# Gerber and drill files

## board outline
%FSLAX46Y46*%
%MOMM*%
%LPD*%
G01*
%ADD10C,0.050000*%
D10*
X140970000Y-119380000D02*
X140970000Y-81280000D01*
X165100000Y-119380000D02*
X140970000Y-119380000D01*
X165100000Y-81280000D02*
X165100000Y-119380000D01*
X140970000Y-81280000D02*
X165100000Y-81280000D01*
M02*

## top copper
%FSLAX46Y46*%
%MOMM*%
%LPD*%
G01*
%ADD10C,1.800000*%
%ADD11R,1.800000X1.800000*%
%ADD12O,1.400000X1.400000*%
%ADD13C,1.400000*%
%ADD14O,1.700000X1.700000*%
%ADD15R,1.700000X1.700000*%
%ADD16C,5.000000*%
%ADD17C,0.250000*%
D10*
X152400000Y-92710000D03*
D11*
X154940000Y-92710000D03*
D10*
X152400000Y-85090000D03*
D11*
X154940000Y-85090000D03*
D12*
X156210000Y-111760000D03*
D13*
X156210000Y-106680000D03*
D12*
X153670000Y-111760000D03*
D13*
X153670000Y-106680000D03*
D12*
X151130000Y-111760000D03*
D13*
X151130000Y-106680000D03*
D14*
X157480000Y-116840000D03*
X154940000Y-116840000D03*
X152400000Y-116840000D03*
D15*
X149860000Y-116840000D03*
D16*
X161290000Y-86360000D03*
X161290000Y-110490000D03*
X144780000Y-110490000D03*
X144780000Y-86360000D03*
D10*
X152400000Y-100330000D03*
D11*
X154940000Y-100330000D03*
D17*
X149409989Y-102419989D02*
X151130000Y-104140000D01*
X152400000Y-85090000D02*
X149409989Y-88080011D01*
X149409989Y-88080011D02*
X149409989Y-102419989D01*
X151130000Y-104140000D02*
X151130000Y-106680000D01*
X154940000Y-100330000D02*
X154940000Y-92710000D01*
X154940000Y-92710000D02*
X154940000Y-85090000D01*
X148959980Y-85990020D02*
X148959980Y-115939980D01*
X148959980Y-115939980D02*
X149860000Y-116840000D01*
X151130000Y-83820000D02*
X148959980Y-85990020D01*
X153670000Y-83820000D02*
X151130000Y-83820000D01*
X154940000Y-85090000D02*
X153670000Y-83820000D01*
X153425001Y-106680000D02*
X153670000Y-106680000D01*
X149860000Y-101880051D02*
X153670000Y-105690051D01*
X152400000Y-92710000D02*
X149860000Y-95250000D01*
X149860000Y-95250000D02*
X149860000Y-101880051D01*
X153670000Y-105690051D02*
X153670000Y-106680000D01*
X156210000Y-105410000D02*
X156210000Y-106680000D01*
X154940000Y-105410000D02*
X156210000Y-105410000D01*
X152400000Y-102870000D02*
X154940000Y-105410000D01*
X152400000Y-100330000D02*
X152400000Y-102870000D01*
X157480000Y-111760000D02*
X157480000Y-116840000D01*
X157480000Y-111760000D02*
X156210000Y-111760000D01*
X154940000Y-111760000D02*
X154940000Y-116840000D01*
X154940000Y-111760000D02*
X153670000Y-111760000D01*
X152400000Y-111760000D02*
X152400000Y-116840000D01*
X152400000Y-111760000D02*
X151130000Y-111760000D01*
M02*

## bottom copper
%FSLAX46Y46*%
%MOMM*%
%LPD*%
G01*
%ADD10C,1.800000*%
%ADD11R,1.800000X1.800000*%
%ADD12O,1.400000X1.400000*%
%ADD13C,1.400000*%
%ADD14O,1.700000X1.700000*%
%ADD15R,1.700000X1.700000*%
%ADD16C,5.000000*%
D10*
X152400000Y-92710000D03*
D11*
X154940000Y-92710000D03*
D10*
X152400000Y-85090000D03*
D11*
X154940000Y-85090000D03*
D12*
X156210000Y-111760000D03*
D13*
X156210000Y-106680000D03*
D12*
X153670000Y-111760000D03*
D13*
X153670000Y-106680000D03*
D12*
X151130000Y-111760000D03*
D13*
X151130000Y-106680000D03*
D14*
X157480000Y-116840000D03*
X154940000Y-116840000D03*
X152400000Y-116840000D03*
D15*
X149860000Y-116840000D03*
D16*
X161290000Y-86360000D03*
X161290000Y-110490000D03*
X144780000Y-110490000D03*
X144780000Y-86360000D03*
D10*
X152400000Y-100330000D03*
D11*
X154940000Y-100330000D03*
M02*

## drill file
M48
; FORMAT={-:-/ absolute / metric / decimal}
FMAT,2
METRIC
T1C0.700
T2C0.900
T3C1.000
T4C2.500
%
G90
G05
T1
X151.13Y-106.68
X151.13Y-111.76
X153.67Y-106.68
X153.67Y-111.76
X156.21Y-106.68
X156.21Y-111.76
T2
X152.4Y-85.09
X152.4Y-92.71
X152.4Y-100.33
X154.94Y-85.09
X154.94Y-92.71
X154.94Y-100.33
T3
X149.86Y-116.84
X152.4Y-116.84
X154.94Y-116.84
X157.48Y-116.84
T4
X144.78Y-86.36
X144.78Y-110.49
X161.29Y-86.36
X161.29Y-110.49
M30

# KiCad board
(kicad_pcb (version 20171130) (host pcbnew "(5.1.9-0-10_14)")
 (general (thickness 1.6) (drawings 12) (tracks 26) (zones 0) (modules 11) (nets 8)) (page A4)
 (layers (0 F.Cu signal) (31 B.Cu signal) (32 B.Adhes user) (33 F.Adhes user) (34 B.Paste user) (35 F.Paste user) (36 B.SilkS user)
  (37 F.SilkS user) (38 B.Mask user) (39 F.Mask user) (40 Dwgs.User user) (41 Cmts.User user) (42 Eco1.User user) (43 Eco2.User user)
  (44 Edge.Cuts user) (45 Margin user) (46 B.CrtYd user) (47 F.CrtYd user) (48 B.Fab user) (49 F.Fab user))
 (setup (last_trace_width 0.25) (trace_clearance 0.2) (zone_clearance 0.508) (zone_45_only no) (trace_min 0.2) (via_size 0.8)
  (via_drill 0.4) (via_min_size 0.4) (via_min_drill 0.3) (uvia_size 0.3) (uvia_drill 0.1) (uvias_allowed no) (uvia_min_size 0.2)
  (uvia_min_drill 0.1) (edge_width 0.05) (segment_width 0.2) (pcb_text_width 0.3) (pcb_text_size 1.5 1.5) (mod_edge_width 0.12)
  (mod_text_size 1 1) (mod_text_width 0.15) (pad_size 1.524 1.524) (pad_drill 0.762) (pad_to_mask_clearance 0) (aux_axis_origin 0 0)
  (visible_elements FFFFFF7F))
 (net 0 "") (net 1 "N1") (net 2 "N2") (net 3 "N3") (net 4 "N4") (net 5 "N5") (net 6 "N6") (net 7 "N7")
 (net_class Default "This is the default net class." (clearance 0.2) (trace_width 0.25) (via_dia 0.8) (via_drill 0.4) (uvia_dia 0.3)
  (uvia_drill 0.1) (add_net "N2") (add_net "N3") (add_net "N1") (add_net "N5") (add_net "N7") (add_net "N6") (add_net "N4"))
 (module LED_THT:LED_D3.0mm (layer F.Cu) (at 154.94 92.71 180)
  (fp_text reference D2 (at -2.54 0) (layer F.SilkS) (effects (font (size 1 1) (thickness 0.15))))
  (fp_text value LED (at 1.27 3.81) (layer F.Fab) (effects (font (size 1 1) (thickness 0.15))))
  (pad 2 thru_hole circle (at 2.54 0 180) (size 1.8 1.8) (drill 0.9) (layers *.Cu *.Mask) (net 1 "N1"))
  (pad 1 thru_hole rect (at 0 0 180) (size 1.8 1.8) (drill 0.9) (layers *.Cu *.Mask) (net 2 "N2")))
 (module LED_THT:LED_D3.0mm (layer F.Cu) (at 154.94 85.09 180)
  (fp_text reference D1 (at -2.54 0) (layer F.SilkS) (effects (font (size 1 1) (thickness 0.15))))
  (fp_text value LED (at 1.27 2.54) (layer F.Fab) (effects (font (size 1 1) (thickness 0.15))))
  (pad 2 thru_hole circle (at 2.54 0 180) (size 1.8 1.8) (drill 0.9) (layers *.Cu *.Mask) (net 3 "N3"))
  (pad 1 thru_hole rect (at 0 0 180) (size 1.8 1.8) (drill 0.9) (layers *.Cu *.Mask) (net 2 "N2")))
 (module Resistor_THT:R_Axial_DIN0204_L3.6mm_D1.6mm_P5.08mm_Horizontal (layer F.Cu) (at 156.21 106.68 270)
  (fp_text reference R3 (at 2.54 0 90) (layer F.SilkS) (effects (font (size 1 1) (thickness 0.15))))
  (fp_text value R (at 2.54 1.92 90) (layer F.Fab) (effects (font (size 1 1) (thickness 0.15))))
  (pad 2 thru_hole oval (at 5.08 0 270) (size 1.4 1.4) (drill 0.7) (layers *.Cu *.Mask) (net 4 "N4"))
  (pad 1 thru_hole circle (at 0 0 270) (size 1.4 1.4) (drill 0.7) (layers *.Cu *.Mask) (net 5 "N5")))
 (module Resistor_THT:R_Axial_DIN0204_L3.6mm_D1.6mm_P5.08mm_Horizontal (layer F.Cu) (at 153.67 106.68 270)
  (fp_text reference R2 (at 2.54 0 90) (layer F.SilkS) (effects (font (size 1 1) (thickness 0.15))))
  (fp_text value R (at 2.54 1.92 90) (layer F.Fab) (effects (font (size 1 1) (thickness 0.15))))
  (pad 2 thru_hole oval (at 5.08 0 270) (size 1.4 1.4) (drill 0.7) (layers *.Cu *.Mask) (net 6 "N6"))
  (pad 1 thru_hole circle (at 0 0 270) (size 1.4 1.4) (drill 0.7) (layers *.Cu *.Mask) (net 1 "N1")))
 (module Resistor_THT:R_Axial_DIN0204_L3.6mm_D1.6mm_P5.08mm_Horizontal (layer F.Cu) (at 151.13 106.68 270)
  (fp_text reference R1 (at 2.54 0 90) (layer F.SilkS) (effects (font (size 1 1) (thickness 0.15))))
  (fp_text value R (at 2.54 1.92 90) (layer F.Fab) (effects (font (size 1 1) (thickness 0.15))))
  (pad 2 thru_hole oval (at 5.08 0 270) (size 1.4 1.4) (drill 0.7) (layers *.Cu *.Mask) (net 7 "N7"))
  (pad 1 thru_hole circle (at 0 0 270) (size 1.4 1.4) (drill 0.7) (layers *.Cu *.Mask) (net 3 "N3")))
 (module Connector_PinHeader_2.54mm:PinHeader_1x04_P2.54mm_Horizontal (layer B.Cu) (at 149.86 116.84 270)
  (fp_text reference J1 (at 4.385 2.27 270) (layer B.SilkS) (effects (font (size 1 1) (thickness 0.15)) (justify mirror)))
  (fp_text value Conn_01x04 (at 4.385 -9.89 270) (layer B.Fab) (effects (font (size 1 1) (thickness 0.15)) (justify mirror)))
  (pad 4 thru_hole oval (at 0 -7.62 270) (size 1.7 1.7) (drill 1) (layers *.Cu *.Mask) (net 4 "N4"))
  (pad 3 thru_hole oval (at 0 -5.08 270) (size 1.7 1.7) (drill 1) (layers *.Cu *.Mask) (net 6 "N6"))
  (pad 2 thru_hole oval (at 0 -2.54 270) (size 1.7 1.7) (drill 1) (layers *.Cu *.Mask) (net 7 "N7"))
  (pad 1 thru_hole rect (at 0 0 270) (size 1.7 1.7) (drill 1) (layers *.Cu *.Mask) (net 2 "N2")))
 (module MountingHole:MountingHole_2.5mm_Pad (layer F.Cu) (at 161.29 86.36)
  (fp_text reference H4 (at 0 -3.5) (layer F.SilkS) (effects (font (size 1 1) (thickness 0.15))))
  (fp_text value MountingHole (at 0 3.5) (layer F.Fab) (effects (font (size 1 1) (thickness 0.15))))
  (pad 1 thru_hole circle (at 0 0) (size 5 5) (drill 2.5) (layers *.Cu *.Mask)))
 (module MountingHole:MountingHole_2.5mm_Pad (layer F.Cu) (at 161.29 110.49)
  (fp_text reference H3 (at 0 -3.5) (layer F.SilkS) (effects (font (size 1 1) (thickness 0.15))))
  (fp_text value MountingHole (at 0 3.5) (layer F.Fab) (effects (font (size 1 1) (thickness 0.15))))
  (pad 1 thru_hole circle (at 0 0) (size 5 5) (drill 2.5) (layers *.Cu *.Mask)))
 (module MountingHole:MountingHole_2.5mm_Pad (layer F.Cu) (at 144.78 110.49)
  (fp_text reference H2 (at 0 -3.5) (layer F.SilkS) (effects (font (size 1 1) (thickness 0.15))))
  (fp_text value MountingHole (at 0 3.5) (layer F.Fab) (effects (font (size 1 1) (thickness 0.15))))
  (pad 1 thru_hole circle (at 0 0) (size 5 5) (drill 2.5) (layers *.Cu *.Mask)))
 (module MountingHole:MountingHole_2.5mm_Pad (layer F.Cu) (at 144.78 86.36)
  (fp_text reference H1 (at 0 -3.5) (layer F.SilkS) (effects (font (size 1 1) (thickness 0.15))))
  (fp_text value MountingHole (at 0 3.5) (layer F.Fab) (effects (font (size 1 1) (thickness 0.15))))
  (pad 1 thru_hole circle (at 0 0) (size 5 5) (drill 2.5) (layers *.Cu *.Mask)))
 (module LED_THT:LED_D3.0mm (layer F.Cu) (at 154.94 100.33 180)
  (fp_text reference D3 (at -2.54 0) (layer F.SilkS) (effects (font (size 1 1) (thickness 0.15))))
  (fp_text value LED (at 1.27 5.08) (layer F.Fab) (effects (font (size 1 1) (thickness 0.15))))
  (pad 2 thru_hole circle (at 2.54 0 180) (size 1.8 1.8) (drill 0.9) (layers *.Cu *.Mask) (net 5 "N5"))
  (pad 1 thru_hole rect (at 0 0 180) (size 1.8 1.8) (drill 0.9) (layers *.Cu *.Mask) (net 2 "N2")))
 (gr_line (start 140.97 119.38) (end 140.97 81.28) (layer Edge.Cuts) (width 0.05))
 (gr_line (start 165.1 119.38) (end 140.97 119.38) (layer Edge.Cuts) (width 0.05))
 (gr_line (start 165.1 81.28) (end 165.1 119.38) (layer Edge.Cuts) (width 0.05))
 (gr_line (start 140.97 81.28) (end 165.1 81.28) (layer Edge.Cuts) (width 0.05))
 (segment (start 149.409989 102.419989) (end 151.13 104.14) (width 0.25) (layer F.Cu) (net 3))
 (segment (start 152.4 85.09) (end 149.409989 88.080011) (width 0.25) (layer F.Cu) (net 3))
 (segment (start 149.409989 88.080011) (end 149.409989 102.419989) (width 0.25) (layer F.Cu) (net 3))
 (segment (start 151.13 104.14) (end 151.13 106.68) (width 0.25) (layer F.Cu) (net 3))
 (segment (start 154.94 100.33) (end 154.94 92.71) (width 0.25) (layer F.Cu) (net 2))
 (segment (start 154.94 92.71) (end 154.94 85.09) (width 0.25) (layer F.Cu) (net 2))
 (segment (start 148.95998 85.99002) (end 148.95998 115.93998) (width 0.25) (layer F.Cu) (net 2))
 (segment (start 148.95998 115.93998) (end 149.86 116.84) (width 0.25) (layer F.Cu) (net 2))
 (segment (start 151.13 83.82) (end 148.95998 85.99002) (width 0.25) (layer F.Cu) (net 2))
 (segment (start 153.67 83.82) (end 151.13 83.82) (width 0.25) (layer F.Cu) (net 2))
 (segment (start 154.94 85.09) (end 153.67 83.82) (width 0.25) (layer F.Cu) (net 2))
 (segment (start 153.425001 106.68) (end 153.67 106.68) (width 0.25) (layer F.Cu) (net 1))
 (segment (start 149.86 101.880051) (end 153.67 105.690051) (width 0.25) (layer F.Cu) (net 1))
 (segment (start 152.4 92.71) (end 149.86 95.25) (width 0.25) (layer F.Cu) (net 1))
 (segment (start 149.86 95.25) (end 149.86 101.880051) (width 0.25) (layer F.Cu) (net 1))
 (segment (start 153.67 105.690051) (end 153.67 106.68) (width 0.25) (layer F.Cu) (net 1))
 (segment (start 156.21 105.41) (end 156.21 106.68) (width 0.25) (layer F.Cu) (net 5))
 (segment (start 154.94 105.41) (end 156.21 105.41) (width 0.25) (layer F.Cu) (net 5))
 (segment (start 152.4 102.87) (end 154.94 105.41) (width 0.25) (layer F.Cu) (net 5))
 (segment (start 152.4 100.33) (end 152.4 102.87) (width 0.25) (layer F.Cu) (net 5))
 (segment (start 157.48 111.76) (end 157.48 116.84) (width 0.25) (layer F.Cu) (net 4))
 (segment (start 157.48 111.76) (end 156.21 111.76) (width 0.25) (layer F.Cu) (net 4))
 (segment (start 154.94 111.76) (end 154.94 116.84) (width 0.25) (layer F.Cu) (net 6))
 (segment (start 154.94 111.76) (end 153.67 111.76) (width 0.25) (layer F.Cu) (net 6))
 (segment (start 152.4 111.76) (end 152.4 116.84) (width 0.25) (layer F.Cu) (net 7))
 (segment (start 152.4 111.76) (end 151.13 111.76) (width 0.25) (layer F.Cu) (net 7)))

